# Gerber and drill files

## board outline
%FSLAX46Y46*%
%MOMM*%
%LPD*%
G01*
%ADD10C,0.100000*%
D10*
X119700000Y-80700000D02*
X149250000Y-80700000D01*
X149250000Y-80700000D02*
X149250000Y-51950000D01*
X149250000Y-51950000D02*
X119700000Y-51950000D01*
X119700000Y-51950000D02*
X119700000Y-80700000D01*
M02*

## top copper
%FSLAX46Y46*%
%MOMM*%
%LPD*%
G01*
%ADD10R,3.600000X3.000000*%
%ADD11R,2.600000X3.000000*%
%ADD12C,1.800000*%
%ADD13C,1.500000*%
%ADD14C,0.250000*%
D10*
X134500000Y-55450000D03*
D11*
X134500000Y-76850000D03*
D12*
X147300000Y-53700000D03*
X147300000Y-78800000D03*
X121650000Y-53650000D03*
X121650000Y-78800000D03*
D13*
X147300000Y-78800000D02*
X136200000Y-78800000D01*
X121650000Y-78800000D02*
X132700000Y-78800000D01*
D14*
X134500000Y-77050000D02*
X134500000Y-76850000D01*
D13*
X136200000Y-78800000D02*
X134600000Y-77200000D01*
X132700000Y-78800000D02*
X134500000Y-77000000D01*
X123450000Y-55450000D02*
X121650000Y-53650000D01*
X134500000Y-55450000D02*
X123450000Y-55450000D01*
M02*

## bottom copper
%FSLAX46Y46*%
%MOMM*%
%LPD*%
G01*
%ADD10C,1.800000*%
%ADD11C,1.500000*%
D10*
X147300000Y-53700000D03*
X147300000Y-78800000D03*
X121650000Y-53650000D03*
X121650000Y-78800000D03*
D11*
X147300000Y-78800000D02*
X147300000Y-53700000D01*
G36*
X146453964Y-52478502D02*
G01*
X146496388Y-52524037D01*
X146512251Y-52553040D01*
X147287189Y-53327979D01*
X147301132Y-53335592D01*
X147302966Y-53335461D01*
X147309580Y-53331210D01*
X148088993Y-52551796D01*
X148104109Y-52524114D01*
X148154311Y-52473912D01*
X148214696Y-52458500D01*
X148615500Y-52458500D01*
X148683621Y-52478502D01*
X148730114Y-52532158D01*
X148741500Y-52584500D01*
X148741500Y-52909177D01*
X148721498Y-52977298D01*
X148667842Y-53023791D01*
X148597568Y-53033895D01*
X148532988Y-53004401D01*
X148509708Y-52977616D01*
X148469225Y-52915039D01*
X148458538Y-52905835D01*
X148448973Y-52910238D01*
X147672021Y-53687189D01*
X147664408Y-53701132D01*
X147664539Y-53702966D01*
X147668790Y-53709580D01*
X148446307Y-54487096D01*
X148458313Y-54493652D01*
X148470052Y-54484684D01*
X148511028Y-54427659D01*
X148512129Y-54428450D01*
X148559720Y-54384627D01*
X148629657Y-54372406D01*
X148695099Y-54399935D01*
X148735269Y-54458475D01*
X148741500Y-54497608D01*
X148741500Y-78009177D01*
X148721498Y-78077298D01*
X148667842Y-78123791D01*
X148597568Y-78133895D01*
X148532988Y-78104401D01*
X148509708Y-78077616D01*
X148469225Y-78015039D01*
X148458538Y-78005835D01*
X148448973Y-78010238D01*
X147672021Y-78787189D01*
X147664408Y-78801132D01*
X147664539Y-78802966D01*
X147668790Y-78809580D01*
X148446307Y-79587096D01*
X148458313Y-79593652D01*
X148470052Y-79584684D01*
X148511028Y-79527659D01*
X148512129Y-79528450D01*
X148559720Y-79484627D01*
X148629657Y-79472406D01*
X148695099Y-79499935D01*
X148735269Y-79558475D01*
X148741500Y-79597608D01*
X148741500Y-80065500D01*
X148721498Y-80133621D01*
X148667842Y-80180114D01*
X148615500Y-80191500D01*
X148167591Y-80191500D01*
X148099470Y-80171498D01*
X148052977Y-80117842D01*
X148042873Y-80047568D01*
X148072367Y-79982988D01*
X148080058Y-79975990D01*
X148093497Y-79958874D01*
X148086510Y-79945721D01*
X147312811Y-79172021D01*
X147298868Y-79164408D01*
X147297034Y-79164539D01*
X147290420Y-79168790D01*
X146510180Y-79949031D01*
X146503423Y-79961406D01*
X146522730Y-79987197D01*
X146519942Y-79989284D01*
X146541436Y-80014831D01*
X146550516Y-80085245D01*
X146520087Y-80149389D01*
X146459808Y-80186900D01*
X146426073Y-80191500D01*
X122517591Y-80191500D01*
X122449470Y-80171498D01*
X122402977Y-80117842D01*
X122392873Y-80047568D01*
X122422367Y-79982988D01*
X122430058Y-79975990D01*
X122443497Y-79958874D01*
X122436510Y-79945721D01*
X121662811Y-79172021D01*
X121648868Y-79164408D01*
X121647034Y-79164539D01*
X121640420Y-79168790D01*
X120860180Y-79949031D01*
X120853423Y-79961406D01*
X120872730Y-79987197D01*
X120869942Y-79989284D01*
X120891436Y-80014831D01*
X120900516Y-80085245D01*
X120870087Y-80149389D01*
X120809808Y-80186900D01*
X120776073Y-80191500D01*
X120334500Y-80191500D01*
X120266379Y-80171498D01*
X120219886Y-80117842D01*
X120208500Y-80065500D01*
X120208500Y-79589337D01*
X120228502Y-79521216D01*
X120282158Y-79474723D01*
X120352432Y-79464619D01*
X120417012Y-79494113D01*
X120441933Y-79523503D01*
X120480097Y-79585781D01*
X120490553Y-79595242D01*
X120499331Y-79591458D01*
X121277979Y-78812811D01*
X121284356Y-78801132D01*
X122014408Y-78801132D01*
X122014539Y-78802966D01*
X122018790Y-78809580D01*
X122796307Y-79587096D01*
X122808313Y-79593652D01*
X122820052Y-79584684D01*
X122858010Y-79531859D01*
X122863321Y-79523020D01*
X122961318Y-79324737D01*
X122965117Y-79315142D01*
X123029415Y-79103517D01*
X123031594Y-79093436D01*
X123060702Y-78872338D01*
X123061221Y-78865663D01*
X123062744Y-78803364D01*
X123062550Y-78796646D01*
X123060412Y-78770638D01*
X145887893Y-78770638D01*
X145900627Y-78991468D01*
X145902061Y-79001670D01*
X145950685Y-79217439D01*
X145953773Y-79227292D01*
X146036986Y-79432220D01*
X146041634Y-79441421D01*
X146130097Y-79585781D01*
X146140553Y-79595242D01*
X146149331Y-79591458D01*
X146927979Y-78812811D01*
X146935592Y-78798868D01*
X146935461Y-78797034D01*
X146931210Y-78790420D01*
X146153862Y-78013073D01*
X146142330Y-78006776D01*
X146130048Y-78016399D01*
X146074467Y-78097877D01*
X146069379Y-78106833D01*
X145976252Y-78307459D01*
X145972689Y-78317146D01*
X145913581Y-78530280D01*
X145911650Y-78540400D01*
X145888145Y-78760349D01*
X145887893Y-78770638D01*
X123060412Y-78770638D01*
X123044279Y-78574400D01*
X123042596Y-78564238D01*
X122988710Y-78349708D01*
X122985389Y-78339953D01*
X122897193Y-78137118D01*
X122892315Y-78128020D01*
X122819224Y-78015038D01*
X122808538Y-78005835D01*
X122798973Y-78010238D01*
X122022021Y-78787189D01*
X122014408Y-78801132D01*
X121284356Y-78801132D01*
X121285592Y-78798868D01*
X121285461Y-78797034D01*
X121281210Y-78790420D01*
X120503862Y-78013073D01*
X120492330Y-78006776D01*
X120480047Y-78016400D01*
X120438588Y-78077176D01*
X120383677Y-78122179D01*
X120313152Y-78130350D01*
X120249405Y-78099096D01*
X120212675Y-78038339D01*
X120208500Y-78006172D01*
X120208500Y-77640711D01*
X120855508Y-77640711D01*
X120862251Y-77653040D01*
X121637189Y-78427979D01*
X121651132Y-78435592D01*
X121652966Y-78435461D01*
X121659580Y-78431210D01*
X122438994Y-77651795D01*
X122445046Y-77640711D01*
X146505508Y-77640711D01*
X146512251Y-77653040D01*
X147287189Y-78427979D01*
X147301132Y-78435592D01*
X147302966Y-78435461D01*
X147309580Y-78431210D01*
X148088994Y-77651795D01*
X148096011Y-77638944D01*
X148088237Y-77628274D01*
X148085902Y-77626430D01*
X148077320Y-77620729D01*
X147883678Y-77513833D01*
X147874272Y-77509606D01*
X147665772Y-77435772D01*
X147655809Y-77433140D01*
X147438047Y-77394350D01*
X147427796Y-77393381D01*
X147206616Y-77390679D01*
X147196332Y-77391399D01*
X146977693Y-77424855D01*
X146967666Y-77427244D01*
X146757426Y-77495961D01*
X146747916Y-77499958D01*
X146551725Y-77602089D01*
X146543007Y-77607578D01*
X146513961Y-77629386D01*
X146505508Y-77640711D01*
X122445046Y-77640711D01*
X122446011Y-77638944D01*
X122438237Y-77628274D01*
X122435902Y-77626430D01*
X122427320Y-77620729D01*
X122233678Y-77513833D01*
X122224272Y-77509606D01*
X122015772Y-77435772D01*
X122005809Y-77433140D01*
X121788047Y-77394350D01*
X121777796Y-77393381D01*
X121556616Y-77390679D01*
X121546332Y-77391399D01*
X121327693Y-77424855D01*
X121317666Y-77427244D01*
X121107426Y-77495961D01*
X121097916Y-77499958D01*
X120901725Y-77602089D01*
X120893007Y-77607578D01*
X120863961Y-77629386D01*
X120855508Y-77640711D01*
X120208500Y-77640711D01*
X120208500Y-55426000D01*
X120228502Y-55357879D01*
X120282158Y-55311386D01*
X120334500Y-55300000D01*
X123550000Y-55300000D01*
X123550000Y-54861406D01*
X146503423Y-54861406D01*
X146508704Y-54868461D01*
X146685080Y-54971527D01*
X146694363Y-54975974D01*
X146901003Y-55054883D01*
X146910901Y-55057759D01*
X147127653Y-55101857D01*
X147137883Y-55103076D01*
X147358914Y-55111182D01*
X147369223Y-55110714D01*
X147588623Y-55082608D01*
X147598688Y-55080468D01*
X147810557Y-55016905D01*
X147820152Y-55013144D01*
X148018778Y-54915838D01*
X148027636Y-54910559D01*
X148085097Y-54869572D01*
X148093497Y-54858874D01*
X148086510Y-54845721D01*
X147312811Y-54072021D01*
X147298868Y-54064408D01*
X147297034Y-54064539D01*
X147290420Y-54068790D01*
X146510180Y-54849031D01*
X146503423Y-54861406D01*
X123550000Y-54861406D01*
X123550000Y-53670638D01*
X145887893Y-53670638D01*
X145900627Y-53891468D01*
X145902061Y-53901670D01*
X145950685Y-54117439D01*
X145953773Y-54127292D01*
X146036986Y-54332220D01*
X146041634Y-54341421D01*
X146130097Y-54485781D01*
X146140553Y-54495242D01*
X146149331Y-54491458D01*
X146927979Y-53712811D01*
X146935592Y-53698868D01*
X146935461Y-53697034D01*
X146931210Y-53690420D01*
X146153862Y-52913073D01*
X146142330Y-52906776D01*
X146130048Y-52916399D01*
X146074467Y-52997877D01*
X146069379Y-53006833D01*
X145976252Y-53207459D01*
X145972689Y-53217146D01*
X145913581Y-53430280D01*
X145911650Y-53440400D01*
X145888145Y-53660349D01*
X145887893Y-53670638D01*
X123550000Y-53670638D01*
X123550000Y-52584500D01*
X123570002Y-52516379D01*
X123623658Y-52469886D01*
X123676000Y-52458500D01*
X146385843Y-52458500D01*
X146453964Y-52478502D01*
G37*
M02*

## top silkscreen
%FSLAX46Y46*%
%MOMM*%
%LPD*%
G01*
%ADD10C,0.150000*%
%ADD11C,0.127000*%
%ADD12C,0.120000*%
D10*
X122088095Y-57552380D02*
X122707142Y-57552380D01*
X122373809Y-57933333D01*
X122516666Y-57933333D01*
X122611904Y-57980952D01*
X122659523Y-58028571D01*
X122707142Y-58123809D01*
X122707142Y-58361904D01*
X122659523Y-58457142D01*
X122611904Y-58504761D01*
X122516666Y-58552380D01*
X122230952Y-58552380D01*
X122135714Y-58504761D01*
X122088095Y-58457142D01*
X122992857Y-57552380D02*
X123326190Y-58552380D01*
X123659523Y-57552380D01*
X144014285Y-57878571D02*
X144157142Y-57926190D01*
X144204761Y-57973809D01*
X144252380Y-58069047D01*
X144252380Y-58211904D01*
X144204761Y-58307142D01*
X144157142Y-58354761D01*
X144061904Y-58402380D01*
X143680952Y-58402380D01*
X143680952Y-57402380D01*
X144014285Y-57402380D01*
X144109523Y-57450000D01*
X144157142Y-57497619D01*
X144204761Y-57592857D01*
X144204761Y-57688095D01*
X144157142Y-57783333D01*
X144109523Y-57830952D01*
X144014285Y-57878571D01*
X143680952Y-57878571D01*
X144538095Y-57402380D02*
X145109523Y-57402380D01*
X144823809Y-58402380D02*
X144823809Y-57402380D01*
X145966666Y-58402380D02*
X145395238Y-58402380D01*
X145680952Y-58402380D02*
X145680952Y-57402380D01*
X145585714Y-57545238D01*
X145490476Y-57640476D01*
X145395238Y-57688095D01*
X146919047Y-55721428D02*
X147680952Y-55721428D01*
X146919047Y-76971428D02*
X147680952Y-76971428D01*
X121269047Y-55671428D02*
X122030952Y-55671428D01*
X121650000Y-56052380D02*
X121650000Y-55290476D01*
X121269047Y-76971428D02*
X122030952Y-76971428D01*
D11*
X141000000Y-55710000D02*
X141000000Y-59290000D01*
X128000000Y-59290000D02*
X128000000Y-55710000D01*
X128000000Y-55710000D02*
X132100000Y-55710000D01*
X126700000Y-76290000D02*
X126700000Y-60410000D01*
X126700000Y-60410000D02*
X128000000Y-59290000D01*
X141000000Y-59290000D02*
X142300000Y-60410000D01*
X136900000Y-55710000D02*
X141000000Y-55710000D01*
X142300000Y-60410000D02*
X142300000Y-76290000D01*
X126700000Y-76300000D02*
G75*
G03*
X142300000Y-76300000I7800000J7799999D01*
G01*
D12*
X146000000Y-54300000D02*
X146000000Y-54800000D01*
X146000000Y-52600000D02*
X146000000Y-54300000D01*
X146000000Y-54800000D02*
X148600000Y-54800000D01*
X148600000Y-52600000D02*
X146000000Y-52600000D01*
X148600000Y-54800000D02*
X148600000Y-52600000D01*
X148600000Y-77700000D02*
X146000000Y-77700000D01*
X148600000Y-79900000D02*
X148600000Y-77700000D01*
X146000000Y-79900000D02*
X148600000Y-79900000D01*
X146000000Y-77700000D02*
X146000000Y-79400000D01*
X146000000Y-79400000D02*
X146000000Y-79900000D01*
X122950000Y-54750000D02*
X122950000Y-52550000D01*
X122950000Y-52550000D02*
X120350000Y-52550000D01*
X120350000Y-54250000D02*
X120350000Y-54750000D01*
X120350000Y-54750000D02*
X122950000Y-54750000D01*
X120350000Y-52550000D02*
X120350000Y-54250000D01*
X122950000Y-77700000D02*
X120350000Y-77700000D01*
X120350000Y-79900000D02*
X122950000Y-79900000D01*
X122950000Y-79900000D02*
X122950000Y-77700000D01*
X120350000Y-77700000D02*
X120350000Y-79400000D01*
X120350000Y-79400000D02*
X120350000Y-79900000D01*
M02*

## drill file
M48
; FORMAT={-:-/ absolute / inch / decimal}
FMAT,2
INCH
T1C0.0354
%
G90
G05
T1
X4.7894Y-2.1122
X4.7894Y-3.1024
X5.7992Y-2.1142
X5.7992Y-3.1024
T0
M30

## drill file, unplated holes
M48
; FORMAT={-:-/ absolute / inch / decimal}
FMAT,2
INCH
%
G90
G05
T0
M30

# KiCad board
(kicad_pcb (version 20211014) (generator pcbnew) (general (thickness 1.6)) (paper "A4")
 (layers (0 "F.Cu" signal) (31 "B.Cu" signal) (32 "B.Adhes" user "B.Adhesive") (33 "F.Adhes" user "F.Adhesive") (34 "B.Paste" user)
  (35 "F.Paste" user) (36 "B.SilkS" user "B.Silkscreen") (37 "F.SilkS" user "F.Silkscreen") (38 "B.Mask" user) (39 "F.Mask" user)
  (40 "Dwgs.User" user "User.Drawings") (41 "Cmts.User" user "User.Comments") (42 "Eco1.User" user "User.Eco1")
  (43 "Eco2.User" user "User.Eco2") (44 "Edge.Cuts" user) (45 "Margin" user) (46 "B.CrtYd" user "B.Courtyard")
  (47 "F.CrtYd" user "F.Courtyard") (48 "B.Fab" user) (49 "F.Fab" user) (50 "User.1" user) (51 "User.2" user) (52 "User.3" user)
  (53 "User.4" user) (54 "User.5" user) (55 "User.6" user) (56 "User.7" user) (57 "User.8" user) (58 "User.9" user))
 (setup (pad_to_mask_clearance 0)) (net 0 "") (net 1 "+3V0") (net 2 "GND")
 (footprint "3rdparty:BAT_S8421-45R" (layer "F.Cu") (at 134.5 68.35 180)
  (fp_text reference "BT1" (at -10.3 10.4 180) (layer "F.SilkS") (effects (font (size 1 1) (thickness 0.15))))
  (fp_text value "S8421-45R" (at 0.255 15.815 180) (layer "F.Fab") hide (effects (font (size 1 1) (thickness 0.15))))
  (fp_line (start -6.5 12.64) (end -6.5 9.06) (layer "F.SilkS") (width 0.127))
  (fp_line (start 6.5 9.06) (end 6.5 12.64) (layer "F.SilkS") (width 0.127))
  (fp_line (start 6.5 12.64) (end 2.4 12.64) (layer "F.SilkS") (width 0.127))
  (fp_line (start 7.8 -7.94) (end 7.8 7.94) (layer "F.SilkS") (width 0.127))
  (fp_line (start 7.8 7.94) (end 6.5 9.06) (layer "F.SilkS") (width 0.127))
  (fp_line (start -6.5 9.06) (end -7.8 7.94) (layer "F.SilkS") (width 0.127))
  (fp_line (start -2.4 12.64) (end -6.5 12.64) (layer "F.SilkS") (width 0.127))
  (fp_line (start -7.8 7.94) (end -7.8 -7.94) (layer "F.SilkS") (width 0.127))
  (fp_arc (start -7.8 -7.95) (mid 0 -11.180866) (end 7.8 -7.95) (layer "F.SilkS") (width 0.127))
  (pad "+" smd rect locked (at 0 12.9 180) (size 3.6 3) (layers "F.Cu" "F.Paste" "F.Mask") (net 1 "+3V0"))
  (pad "-" smd rect locked (at 0 -8.5 180) (size 2.6 3) (layers "F.Cu" "F.Paste" "F.Mask") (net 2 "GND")))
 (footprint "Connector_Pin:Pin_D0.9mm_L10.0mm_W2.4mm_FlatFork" (layer "F.Cu") (at 147.3 53.7)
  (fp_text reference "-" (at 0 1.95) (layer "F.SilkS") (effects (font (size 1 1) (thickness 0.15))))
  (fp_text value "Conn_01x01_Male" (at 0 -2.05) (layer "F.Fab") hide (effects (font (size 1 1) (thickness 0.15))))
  (fp_line (start -1.3 0.6) (end -1.3 1.1) (layer "F.SilkS") (width 0.12))
  (fp_line (start -1.3 -1.1) (end -1.3 0.6) (layer "F.SilkS") (width 0.12))
  (fp_line (start -1.3 1.1) (end 1.3 1.1) (layer "F.SilkS") (width 0.12))
  (fp_line (start 1.3 -1.1) (end -1.3 -1.1) (layer "F.SilkS") (width 0.12))
  (fp_line (start 1.3 1.1) (end 1.3 -1.1) (layer "F.SilkS") (width 0.12))
  (pad "1" thru_hole circle (at 0 0) (size 1.8 1.8) (drill 0.9) (layers *.Cu *.Mask) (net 2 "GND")))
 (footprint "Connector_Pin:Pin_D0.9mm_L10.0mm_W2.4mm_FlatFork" (layer "F.Cu") (at 147.3 78.8)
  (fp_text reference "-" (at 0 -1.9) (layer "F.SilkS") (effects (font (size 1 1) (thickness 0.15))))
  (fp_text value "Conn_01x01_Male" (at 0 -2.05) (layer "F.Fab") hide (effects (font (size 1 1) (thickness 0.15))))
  (fp_line (start 1.3 -1.1) (end -1.3 -1.1) (layer "F.SilkS") (width 0.12))
  (fp_line (start 1.3 1.1) (end 1.3 -1.1) (layer "F.SilkS") (width 0.12))
  (fp_line (start -1.3 1.1) (end 1.3 1.1) (layer "F.SilkS") (width 0.12))
  (fp_line (start -1.3 -1.1) (end -1.3 0.6) (layer "F.SilkS") (width 0.12))
  (fp_line (start -1.3 0.6) (end -1.3 1.1) (layer "F.SilkS") (width 0.12))
  (pad "1" thru_hole circle (at 0 0) (size 1.8 1.8) (drill 0.9) (layers *.Cu *.Mask) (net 2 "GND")))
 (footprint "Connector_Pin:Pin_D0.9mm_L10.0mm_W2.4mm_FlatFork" (layer "F.Cu") (at 121.65 53.65)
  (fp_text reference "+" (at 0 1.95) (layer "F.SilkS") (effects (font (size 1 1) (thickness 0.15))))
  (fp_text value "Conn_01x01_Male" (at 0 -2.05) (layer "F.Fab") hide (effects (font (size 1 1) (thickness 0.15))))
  (fp_line (start 1.3 1.1) (end 1.3 -1.1) (layer "F.SilkS") (width 0.12))
  (fp_line (start 1.3 -1.1) (end -1.3 -1.1) (layer "F.SilkS") (width 0.12))
  (fp_line (start -1.3 0.6) (end -1.3 1.1) (layer "F.SilkS") (width 0.12))
  (fp_line (start -1.3 1.1) (end 1.3 1.1) (layer "F.SilkS") (width 0.12))
  (fp_line (start -1.3 -1.1) (end -1.3 0.6) (layer "F.SilkS") (width 0.12))
  (pad "1" thru_hole circle (at 0 0) (size 1.8 1.8) (drill 0.9) (layers *.Cu *.Mask) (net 1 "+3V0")))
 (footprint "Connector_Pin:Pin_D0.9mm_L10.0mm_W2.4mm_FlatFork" (layer "F.Cu") (at 121.65 78.8)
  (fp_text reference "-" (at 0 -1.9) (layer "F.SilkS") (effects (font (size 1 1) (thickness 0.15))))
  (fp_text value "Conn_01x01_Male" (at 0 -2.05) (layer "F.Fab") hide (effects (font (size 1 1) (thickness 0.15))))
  (fp_line (start 1.3 -1.1) (end -1.3 -1.1) (layer "F.SilkS") (width 0.12))
  (fp_line (start -1.3 1.1) (end 1.3 1.1) (layer "F.SilkS") (width 0.12))
  (fp_line (start 1.3 1.1) (end 1.3 -1.1) (layer "F.SilkS") (width 0.12))
  (fp_line (start -1.3 -1.1) (end -1.3 0.6) (layer "F.SilkS") (width 0.12))
  (fp_line (start -1.3 0.6) (end -1.3 1.1) (layer "F.SilkS") (width 0.12))
  (pad "1" thru_hole circle (at 0 0) (size 1.8 1.8) (drill 0.9) (layers *.Cu *.Mask) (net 2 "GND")))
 (gr_rect (start 119.7 80.7) (end 149.25 51.95) (layer "Edge.Cuts") (width 0.1) (fill none))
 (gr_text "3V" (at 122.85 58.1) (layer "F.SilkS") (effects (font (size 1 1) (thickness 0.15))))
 (segment (start 147.3 78.8) (end 136.2 78.8) (width 1.5) (layer "F.Cu") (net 2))
 (segment (start 121.65 78.8) (end 132.7 78.8) (width 1.5) (layer "F.Cu") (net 2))
 (segment (start 134.5 77.05) (end 134.5 76.85) (width 0.25) (layer "F.Cu") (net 2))
 (segment (start 136.2 78.8) (end 134.6 77.2) (width 1.5) (layer "F.Cu") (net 2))
 (segment (start 132.7 78.8) (end 134.5 77) (width 1.5) (layer "F.Cu") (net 2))
 (segment (start 147.3 78.8) (end 147.3 53.7) (width 1.5) (layer "B.Cu") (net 2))
 (segment (start 123.45 55.45) (end 121.65 53.65) (width 1.5) (layer "F.Cu") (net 1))
 (segment (start 134.5 55.45) (end 123.45 55.45) (width 1.5) (layer "F.Cu") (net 1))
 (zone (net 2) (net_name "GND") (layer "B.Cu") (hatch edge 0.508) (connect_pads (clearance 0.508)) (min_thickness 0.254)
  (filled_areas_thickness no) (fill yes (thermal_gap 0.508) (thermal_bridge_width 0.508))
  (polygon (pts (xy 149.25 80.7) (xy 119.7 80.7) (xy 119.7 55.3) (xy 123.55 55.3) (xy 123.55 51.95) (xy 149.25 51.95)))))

